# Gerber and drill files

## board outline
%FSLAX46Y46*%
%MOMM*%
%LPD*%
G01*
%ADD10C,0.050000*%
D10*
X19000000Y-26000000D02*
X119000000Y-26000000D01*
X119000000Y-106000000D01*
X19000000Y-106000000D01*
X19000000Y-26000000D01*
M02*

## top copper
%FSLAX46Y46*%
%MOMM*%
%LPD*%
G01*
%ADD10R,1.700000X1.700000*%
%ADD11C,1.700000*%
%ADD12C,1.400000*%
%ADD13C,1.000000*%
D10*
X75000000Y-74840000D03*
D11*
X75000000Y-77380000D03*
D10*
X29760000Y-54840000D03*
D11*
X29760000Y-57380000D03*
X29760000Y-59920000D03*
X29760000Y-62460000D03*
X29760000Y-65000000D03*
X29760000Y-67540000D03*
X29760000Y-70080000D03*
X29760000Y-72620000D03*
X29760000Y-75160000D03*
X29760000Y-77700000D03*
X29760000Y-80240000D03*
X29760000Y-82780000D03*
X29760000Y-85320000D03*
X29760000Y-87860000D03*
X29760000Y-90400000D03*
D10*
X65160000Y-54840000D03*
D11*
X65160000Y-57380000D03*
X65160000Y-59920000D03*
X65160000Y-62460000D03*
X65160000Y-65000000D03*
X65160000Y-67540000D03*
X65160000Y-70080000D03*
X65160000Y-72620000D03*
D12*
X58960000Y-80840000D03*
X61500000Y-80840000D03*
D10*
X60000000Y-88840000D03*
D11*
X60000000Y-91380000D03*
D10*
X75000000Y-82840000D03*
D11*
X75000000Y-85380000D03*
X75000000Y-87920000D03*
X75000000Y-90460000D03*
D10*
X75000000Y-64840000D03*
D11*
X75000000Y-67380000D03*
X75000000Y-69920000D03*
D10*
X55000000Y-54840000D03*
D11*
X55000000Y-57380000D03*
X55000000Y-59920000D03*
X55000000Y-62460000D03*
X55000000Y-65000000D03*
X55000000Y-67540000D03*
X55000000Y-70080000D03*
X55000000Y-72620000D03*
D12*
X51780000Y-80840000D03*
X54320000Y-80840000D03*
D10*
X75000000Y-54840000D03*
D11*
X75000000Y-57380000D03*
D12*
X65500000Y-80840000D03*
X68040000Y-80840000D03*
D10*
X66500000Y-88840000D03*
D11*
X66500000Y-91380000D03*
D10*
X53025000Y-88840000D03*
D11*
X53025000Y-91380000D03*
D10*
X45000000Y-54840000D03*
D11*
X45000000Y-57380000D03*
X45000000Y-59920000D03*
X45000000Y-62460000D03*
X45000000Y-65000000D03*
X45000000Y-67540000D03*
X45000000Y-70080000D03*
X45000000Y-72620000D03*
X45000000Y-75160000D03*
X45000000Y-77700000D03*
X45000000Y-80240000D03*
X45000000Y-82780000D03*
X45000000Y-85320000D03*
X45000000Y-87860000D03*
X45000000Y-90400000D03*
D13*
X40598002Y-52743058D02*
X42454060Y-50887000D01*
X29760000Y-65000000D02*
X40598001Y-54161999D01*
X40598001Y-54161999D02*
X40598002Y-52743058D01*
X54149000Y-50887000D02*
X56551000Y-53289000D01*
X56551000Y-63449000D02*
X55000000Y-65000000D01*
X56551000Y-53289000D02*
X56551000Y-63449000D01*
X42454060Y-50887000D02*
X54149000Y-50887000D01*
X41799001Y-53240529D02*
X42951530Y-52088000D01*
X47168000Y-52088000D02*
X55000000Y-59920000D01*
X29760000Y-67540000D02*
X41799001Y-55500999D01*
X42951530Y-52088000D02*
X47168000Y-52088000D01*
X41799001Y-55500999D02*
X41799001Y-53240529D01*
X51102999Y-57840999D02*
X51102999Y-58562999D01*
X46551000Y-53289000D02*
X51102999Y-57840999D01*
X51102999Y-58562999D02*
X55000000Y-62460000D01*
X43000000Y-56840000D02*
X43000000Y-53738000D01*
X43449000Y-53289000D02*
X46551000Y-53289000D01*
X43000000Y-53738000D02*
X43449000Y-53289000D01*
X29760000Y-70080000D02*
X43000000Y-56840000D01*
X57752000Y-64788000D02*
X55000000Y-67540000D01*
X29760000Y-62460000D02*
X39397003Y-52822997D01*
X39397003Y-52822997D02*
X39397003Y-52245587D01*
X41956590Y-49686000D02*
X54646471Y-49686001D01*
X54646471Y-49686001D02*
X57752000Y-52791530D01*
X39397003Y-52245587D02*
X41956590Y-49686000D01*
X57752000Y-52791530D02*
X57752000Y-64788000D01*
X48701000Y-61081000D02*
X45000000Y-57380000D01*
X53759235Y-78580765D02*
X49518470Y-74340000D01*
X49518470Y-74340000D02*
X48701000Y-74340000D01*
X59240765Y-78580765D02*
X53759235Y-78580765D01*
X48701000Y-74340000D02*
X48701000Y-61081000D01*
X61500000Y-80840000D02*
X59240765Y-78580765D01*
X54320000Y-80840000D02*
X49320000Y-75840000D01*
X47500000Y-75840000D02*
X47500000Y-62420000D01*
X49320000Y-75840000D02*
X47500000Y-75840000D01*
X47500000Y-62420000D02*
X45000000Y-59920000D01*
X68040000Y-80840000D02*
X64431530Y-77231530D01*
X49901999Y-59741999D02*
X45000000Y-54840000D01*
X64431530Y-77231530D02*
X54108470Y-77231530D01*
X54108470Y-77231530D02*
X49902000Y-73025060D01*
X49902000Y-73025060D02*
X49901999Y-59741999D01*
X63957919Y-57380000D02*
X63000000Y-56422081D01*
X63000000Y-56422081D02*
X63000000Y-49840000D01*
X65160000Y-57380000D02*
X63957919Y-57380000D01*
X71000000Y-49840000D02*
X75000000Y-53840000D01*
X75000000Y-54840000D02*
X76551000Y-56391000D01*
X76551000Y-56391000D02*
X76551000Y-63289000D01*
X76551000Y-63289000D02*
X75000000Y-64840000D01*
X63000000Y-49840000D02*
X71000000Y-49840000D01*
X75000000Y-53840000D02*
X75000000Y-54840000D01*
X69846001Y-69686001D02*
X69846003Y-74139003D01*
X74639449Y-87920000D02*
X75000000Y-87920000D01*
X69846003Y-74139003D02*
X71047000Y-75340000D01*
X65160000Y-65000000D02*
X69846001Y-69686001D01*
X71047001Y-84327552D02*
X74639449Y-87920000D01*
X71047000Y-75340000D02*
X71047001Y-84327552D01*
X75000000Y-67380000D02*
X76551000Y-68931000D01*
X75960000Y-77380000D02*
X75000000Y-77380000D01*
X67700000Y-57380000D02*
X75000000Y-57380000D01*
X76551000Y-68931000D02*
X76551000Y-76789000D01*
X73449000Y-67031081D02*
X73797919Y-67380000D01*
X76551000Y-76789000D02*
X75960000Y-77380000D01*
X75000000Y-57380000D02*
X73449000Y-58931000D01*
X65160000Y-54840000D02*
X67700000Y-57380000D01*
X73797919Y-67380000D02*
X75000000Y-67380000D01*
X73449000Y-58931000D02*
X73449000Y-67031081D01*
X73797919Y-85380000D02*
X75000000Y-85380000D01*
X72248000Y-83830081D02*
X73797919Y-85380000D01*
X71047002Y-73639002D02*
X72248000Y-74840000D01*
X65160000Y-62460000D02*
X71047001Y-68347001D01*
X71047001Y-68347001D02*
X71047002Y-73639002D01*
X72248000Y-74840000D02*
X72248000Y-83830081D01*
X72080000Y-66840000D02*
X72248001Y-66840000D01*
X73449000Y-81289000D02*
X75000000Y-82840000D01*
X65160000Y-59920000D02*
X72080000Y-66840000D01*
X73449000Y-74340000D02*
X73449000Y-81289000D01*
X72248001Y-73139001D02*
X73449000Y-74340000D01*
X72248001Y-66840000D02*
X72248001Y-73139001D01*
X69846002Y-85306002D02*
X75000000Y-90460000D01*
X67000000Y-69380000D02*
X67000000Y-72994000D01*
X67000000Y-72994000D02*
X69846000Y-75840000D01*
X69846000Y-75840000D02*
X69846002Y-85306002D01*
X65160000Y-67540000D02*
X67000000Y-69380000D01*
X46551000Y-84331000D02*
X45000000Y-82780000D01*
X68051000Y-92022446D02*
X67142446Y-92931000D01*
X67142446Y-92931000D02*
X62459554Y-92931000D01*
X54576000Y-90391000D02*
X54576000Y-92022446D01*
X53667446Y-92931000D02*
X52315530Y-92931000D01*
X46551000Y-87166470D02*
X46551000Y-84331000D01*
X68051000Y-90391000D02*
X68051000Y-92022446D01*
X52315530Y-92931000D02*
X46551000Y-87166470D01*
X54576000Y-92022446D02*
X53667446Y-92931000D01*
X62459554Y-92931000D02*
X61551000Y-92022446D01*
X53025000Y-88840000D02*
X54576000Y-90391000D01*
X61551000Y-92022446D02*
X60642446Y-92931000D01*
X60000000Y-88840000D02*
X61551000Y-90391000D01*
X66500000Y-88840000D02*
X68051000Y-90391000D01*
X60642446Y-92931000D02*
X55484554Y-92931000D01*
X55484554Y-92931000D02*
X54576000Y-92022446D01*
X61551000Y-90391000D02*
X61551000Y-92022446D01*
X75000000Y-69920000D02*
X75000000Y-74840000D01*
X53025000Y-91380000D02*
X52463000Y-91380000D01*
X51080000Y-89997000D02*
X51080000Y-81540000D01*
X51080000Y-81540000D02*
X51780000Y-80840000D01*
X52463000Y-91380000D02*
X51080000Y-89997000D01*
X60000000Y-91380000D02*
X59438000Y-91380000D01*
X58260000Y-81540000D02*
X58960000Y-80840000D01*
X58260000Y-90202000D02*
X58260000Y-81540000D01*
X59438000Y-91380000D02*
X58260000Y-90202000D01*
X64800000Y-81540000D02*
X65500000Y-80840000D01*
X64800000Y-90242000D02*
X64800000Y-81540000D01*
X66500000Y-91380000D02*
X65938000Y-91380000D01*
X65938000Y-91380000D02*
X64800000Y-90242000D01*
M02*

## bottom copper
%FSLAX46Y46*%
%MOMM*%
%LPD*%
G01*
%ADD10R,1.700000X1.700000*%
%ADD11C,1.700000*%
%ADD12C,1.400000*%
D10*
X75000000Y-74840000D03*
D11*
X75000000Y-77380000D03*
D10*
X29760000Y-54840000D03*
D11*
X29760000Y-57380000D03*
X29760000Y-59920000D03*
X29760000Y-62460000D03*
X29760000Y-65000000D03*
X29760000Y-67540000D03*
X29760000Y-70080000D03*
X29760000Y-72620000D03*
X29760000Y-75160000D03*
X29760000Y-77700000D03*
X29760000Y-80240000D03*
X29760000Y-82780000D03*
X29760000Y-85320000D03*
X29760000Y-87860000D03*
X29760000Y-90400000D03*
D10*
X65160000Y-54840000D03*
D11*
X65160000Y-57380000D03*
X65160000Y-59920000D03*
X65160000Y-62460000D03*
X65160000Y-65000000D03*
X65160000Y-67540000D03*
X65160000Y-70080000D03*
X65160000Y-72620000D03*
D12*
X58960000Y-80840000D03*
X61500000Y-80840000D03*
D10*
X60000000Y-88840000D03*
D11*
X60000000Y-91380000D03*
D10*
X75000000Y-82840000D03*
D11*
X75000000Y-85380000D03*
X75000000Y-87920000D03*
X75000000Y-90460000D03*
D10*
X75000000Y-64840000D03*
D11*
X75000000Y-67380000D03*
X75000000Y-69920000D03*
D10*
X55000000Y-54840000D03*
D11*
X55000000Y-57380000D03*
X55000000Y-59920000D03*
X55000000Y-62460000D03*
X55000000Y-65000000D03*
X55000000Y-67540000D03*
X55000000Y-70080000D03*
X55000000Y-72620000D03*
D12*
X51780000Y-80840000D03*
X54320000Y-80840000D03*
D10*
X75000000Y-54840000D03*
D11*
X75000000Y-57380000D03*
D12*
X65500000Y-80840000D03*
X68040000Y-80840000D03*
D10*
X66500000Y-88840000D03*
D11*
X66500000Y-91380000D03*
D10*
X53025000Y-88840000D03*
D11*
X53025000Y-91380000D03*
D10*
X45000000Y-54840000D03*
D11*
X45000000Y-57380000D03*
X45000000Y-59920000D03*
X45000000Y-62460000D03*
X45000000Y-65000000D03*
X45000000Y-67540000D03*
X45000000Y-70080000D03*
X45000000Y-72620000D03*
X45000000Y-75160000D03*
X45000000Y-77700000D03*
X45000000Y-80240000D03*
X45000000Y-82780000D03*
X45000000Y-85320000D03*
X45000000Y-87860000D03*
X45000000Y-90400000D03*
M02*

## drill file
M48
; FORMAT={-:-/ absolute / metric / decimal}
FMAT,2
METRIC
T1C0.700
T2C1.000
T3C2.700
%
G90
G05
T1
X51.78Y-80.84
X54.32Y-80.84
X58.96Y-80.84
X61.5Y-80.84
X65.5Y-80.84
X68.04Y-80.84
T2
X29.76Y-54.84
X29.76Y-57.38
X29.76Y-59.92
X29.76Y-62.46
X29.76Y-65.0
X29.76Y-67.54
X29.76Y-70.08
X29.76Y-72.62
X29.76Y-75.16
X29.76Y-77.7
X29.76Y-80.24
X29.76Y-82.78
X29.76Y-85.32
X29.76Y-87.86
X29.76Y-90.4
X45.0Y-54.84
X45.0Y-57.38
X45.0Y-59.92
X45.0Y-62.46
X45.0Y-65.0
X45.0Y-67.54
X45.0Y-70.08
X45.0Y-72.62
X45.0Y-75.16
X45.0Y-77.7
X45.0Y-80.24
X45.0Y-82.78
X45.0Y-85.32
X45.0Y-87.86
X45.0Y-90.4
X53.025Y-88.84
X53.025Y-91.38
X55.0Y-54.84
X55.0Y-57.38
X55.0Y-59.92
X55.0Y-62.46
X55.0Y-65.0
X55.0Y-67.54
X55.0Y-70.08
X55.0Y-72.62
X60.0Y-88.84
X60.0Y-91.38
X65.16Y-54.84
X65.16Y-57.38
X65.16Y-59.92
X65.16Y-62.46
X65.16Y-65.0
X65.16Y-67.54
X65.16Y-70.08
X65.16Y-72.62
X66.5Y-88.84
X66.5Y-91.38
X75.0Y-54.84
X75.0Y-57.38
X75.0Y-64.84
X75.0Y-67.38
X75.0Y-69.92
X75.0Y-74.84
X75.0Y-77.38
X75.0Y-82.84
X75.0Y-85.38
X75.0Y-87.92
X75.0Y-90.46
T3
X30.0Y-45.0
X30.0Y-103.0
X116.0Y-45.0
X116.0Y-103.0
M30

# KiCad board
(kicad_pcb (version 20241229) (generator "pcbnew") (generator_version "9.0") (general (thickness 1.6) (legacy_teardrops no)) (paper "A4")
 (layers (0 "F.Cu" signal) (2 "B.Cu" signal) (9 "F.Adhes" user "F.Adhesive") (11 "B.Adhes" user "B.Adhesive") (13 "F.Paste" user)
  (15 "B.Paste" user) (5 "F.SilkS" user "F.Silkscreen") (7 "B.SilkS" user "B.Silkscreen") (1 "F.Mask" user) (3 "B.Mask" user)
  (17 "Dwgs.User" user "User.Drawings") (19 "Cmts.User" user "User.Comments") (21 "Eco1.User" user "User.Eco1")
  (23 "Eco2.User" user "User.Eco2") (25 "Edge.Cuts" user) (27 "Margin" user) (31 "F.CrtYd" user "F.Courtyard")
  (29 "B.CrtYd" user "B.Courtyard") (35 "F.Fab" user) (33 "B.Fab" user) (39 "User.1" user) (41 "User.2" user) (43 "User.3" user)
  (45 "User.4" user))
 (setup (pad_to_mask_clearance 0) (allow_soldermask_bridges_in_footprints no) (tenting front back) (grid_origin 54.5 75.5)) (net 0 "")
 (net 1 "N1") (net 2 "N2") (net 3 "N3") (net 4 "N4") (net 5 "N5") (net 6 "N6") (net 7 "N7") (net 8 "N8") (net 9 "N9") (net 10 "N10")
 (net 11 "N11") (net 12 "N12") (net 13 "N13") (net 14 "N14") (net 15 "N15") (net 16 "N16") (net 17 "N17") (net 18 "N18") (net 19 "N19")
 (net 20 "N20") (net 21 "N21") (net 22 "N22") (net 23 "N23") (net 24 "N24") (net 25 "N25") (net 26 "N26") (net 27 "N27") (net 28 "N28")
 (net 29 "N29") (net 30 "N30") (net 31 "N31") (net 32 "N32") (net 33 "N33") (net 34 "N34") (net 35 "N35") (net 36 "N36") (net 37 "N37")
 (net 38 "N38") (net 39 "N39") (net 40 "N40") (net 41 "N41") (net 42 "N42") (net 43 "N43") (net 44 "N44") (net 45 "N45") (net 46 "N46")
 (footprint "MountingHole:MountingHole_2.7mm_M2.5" (layer "F.Cu") (at 30 103)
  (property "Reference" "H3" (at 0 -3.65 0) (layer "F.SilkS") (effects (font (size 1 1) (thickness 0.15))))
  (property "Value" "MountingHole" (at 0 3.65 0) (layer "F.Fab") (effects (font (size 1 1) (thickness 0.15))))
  (pad "" np_thru_hole circle (at 0 0) (size 2.7 2.7) (drill 2.7) (layers "*.Cu" "*.Mask")))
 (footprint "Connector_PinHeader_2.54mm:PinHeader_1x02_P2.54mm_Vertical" (layer "F.Cu") (at 75 74.84)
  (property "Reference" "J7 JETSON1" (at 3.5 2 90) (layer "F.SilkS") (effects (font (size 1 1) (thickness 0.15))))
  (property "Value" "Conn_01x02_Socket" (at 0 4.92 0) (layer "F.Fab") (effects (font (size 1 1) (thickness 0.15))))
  (pad "1" thru_hole rect (at 0 0) (size 1.7 1.7) (drill 1) (layers "*.Cu" "*.Mask") (remove_unused_layers no) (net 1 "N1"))
  (pad "2" thru_hole circle (at 0 2.54) (size 1.7 1.7) (drill 1) (layers "*.Cu" "*.Mask") (remove_unused_layers no) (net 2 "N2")))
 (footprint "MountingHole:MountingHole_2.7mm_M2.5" (layer "F.Cu") (at 30 45)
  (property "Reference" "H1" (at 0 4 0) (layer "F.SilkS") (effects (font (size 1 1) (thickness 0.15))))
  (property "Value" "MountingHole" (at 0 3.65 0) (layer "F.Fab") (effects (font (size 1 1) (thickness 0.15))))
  (pad "" np_thru_hole circle (at 0 0) (size 2.7 2.7) (drill 2.7) (layers "*.Cu" "*.Mask")))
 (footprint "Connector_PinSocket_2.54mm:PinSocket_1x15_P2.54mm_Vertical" (layer "F.Cu") (at 29.76 54.84)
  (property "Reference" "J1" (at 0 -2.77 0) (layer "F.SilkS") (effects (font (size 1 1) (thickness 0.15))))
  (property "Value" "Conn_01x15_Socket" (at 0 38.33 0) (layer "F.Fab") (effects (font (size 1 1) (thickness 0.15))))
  (pad "1" thru_hole rect (at 0 0) (size 1.7 1.7) (drill 1) (layers "*.Cu" "*.Mask") (remove_unused_layers no) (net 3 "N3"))
  (pad "2" thru_hole circle (at 0 2.54) (size 1.7 1.7) (drill 1) (layers "*.Cu" "*.Mask") (remove_unused_layers no) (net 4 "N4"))
  (pad "3" thru_hole circle (at 0 5.08) (size 1.7 1.7) (drill 1) (layers "*.Cu" "*.Mask") (remove_unused_layers no) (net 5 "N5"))
  (pad "4" thru_hole circle (at 0 7.62) (size 1.7 1.7) (drill 1) (layers "*.Cu" "*.Mask") (remove_unused_layers no) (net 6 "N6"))
  (pad "5" thru_hole circle (at 0 10.16) (size 1.7 1.7) (drill 1) (layers "*.Cu" "*.Mask") (remove_unused_layers no) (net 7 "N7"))
  (pad "6" thru_hole circle (at 0 12.7) (size 1.7 1.7) (drill 1) (layers "*.Cu" "*.Mask") (remove_unused_layers no) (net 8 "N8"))
  (pad "7" thru_hole circle (at 0 15.24) (size 1.7 1.7) (drill 1) (layers "*.Cu" "*.Mask") (remove_unused_layers no) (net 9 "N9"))
  (pad "8" thru_hole circle (at 0 17.78) (size 1.7 1.7) (drill 1) (layers "*.Cu" "*.Mask") (remove_unused_layers no) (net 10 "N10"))
  (pad "9" thru_hole circle (at 0 20.32) (size 1.7 1.7) (drill 1) (layers "*.Cu" "*.Mask") (remove_unused_layers no) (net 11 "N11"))
  (pad "10" thru_hole circle (at 0 22.86) (size 1.7 1.7) (drill 1) (layers "*.Cu" "*.Mask") (remove_unused_layers no) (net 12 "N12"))
  (pad "11" thru_hole circle (at 0 25.4) (size 1.7 1.7) (drill 1) (layers "*.Cu" "*.Mask") (remove_unused_layers no) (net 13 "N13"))
  (pad "12" thru_hole circle (at 0 27.94) (size 1.7 1.7) (drill 1) (layers "*.Cu" "*.Mask") (remove_unused_layers no) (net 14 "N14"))
  (pad "13" thru_hole circle (at 0 30.48) (size 1.7 1.7) (drill 1) (layers "*.Cu" "*.Mask") (remove_unused_layers no) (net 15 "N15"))
  (pad "14" thru_hole circle (at 0 33.02) (size 1.7 1.7) (drill 1) (layers "*.Cu" "*.Mask") (remove_unused_layers no) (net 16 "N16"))
  (pad "15" thru_hole circle (at 0 35.56) (size 1.7 1.7) (drill 1) (layers "*.Cu" "*.Mask") (remove_unused_layers no) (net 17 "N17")))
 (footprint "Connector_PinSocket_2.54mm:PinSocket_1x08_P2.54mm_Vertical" (layer "F.Cu") (at 65.16 54.84)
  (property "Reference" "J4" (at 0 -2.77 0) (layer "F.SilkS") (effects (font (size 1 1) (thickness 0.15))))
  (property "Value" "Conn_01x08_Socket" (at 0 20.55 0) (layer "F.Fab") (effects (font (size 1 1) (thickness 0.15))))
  (pad "1" thru_hole rect (at 0 0) (size 1.7 1.7) (drill 1) (layers "*.Cu" "*.Mask") (remove_unused_layers no) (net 2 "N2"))
  (pad "2" thru_hole circle (at 0 2.54) (size 1.7 1.7) (drill 1) (layers "*.Cu" "*.Mask") (remove_unused_layers no) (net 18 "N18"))
  (pad "3" thru_hole circle (at 0 5.08) (size 1.7 1.7) (drill 1) (layers "*.Cu" "*.Mask") (remove_unused_layers no) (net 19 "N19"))
  (pad "4" thru_hole circle (at 0 7.62) (size 1.7 1.7) (drill 1) (layers "*.Cu" "*.Mask") (remove_unused_layers no) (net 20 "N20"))
  (pad "5" thru_hole circle (at 0 10.16) (size 1.7 1.7) (drill 1) (layers "*.Cu" "*.Mask") (remove_unused_layers no) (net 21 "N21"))
  (pad "6" thru_hole circle (at 0 12.7) (size 1.7 1.7) (drill 1) (layers "*.Cu" "*.Mask") (remove_unused_layers no) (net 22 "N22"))
  (pad "7" thru_hole circle (at 0 15.24) (size 1.7 1.7) (drill 1) (layers "*.Cu" "*.Mask") (remove_unused_layers no) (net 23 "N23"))
  (pad "8" thru_hole circle (at 0 17.78) (size 1.7 1.7) (drill 1) (layers "*.Cu" "*.Mask") (remove_unused_layers no) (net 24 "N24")))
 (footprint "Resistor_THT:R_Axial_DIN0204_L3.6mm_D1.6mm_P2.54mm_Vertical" (layer "F.Cu") (at 58.96 80.84)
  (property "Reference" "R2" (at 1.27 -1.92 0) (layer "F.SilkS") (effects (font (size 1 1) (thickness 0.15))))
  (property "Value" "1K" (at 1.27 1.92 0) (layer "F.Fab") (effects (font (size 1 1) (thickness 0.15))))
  (pad "1" thru_hole circle (at 0 0) (size 1.4 1.4) (drill 0.7) (layers "*.Cu" "*.Mask") (remove_unused_layers no) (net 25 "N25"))
  (pad "2" thru_hole circle (at 2.54 0) (size 1.4 1.4) (drill 0.7) (layers "*.Cu" "*.Mask") (remove_unused_layers no) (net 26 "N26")))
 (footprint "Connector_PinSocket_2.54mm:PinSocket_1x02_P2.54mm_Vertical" (layer "F.Cu") (at 60 88.84)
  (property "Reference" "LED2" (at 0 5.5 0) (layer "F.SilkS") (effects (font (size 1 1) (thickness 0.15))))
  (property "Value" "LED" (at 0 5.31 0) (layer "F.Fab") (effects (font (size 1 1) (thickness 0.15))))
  (pad "1" thru_hole rect (at 0 0) (size 1.7 1.7) (drill 1) (layers "*.Cu" "*.Mask") (remove_unused_layers no) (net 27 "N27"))
  (pad "2" thru_hole circle (at 0 2.54) (size 1.7 1.7) (drill 1) (layers "*.Cu" "*.Mask") (remove_unused_layers no) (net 25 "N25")))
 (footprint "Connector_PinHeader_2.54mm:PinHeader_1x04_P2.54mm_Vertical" (layer "F.Cu") (at 75 82.84)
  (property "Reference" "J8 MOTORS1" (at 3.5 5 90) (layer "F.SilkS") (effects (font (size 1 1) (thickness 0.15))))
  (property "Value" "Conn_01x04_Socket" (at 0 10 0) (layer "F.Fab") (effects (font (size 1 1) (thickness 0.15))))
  (pad "1" thru_hole rect (at 0 0) (size 1.7 1.7) (drill 1) (layers "*.Cu" "*.Mask") (remove_unused_layers no) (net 19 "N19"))
  (pad "2" thru_hole circle (at 0 2.54) (size 1.7 1.7) (drill 1) (layers "*.Cu" "*.Mask") (remove_unused_layers no) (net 20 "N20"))
  (pad "3" thru_hole circle (at 0 5.08) (size 1.7 1.7) (drill 1) (layers "*.Cu" "*.Mask") (remove_unused_layers no) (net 21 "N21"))
  (pad "4" thru_hole circle (at 0 7.62) (size 1.7 1.7) (drill 1) (layers "*.Cu" "*.Mask") (remove_unused_layers no) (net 22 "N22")))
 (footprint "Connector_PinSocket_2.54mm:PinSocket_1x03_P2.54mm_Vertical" (layer "F.Cu") (at 75 64.84)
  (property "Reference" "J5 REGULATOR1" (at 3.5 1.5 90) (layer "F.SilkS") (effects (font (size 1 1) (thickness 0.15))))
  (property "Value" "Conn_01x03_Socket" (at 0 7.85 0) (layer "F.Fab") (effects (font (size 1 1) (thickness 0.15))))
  (pad "1" thru_hole rect (at 0 0) (size 1.7 1.7) (drill 1) (layers "*.Cu" "*.Mask") (remove_unused_layers no) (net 18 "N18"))
  (pad "2" thru_hole circle (at 0 2.54) (size 1.7 1.7) (drill 1) (layers "*.Cu" "*.Mask") (remove_unused_layers no) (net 2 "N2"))
  (pad "3" thru_hole circle (at 0 5.08) (size 1.7 1.7) (drill 1) (layers "*.Cu" "*.Mask") (remove_unused_layers no) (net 1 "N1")))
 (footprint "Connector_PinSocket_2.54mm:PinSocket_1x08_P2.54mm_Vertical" (layer "F.Cu") (at 55 54.84)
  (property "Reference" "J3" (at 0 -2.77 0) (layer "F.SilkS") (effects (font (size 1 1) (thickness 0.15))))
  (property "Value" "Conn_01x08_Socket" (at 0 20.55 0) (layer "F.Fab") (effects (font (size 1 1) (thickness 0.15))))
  (pad "1" thru_hole rect (at 0 0) (size 1.7 1.7) (drill 1) (layers "*.Cu" "*.Mask") (remove_unused_layers no) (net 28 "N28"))
  (pad "2" thru_hole circle (at 0 2.54) (size 1.7 1.7) (drill 1) (layers "*.Cu" "*.Mask") (remove_unused_layers no) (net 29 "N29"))
  (pad "3" thru_hole circle (at 0 5.08) (size 1.7 1.7) (drill 1) (layers "*.Cu" "*.Mask") (remove_unused_layers no) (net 8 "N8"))
  (pad "4" thru_hole circle (at 0 7.62) (size 1.7 1.7) (drill 1) (layers "*.Cu" "*.Mask") (remove_unused_layers no) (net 9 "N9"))
  (pad "5" thru_hole circle (at 0 10.16) (size 1.7 1.7) (drill 1) (layers "*.Cu" "*.Mask") (remove_unused_layers no) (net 7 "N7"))
  (pad "6" thru_hole circle (at 0 12.7) (size 1.7 1.7) (drill 1) (layers "*.Cu" "*.Mask") (remove_unused_layers no) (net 6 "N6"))
  (pad "7" thru_hole circle (at 0 15.24) (size 1.7 1.7) (drill 1) (layers "*.Cu" "*.Mask") (remove_unused_layers no) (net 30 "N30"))
  (pad "8" thru_hole circle (at 0 17.78) (size 1.7 1.7) (drill 1) (layers "*.Cu" "*.Mask") (remove_unused_layers no) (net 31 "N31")))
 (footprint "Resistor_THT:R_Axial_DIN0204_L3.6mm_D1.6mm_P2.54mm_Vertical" (layer "F.Cu") (at 51.78 80.84)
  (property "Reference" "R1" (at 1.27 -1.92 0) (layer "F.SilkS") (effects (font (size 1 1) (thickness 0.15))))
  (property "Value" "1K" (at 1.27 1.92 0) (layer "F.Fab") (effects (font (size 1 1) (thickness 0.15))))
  (pad "1" thru_hole circle (at 0 0) (size 1.4 1.4) (drill 0.7) (layers "*.Cu" "*.Mask") (remove_unused_layers no) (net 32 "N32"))
  (pad "2" thru_hole circle (at 2.54 0) (size 1.4 1.4) (drill 0.7) (layers "*.Cu" "*.Mask") (remove_unused_layers no) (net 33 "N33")))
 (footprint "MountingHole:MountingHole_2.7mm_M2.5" (layer "F.Cu") (at 116 45)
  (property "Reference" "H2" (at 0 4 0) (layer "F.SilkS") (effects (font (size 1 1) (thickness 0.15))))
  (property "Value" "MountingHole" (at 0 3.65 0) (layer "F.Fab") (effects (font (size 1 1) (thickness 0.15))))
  (pad "" np_thru_hole circle (at 0 0) (size 2.7 2.7) (drill 2.7) (layers "*.Cu" "*.Mask")))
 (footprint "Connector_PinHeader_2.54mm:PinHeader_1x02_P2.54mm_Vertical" (layer "F.Cu") (at 75 54.84)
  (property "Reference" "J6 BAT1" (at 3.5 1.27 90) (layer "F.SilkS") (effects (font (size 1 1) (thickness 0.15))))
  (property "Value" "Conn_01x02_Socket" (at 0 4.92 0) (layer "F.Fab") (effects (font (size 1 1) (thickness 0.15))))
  (pad "1" thru_hole rect (at 0 0) (size 1.7 1.7) (drill 1) (layers "*.Cu" "*.Mask") (remove_unused_layers no) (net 18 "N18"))
  (pad "2" thru_hole circle (at 0 2.54) (size 1.7 1.7) (drill 1) (layers "*.Cu" "*.Mask") (remove_unused_layers no) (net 2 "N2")))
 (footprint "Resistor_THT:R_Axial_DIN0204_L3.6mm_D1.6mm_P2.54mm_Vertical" (layer "F.Cu") (at 65.5 80.84)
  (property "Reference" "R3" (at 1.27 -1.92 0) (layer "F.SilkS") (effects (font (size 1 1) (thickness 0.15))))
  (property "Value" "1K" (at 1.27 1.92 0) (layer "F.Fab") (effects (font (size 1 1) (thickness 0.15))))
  (pad "1" thru_hole circle (at 0 0) (size 1.4 1.4) (drill 0.7) (layers "*.Cu" "*.Mask") (remove_unused_layers no) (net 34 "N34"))
  (pad "2" thru_hole circle (at 2.54 0) (size 1.4 1.4) (drill 0.7) (layers "*.Cu" "*.Mask") (remove_unused_layers no) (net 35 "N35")))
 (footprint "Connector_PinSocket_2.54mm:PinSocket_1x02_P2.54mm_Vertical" (layer "F.Cu") (at 66.5 88.84)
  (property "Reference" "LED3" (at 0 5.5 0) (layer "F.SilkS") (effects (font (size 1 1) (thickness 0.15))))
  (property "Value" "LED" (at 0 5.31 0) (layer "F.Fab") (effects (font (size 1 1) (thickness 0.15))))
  (pad "1" thru_hole rect (at 0 0) (size 1.7 1.7) (drill 1) (layers "*.Cu" "*.Mask") (remove_unused_layers no) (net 27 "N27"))
  (pad "2" thru_hole circle (at 0 2.54) (size 1.7 1.7) (drill 1) (layers "*.Cu" "*.Mask") (remove_unused_layers no) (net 34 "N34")))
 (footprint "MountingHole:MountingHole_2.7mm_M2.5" (layer "F.Cu") (at 116 103)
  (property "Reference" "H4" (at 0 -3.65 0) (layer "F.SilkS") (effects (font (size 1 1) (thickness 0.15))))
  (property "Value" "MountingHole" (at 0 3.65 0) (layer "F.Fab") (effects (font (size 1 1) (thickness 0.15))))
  (pad "" np_thru_hole circle (at 0 0) (size 2.7 2.7) (drill 2.7) (layers "*.Cu" "*.Mask")))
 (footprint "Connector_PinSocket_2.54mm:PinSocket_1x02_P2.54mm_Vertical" (layer "F.Cu") (at 53.025 88.84)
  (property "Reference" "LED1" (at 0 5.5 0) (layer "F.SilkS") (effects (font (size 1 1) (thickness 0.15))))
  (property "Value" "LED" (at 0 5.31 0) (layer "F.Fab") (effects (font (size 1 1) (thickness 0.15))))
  (pad "1" thru_hole rect (at 0 0) (size 1.7 1.7) (drill 1) (layers "*.Cu" "*.Mask") (remove_unused_layers no) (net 27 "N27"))
  (pad "2" thru_hole circle (at 0 2.54) (size 1.7 1.7) (drill 1) (layers "*.Cu" "*.Mask") (remove_unused_layers no) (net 32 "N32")))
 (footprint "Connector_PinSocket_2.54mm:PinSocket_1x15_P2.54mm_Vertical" (layer "F.Cu") (at 45 54.84)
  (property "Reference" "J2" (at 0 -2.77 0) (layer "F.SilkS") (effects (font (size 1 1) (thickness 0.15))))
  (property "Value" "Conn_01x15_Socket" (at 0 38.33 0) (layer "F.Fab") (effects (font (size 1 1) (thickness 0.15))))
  (pad "1" thru_hole rect (at 0 0) (size 1.7 1.7) (drill 1) (layers "*.Cu" "*.Mask") (remove_unused_layers no) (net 35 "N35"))
  (pad "2" thru_hole circle (at 0 2.54) (size 1.7 1.7) (drill 1) (layers "*.Cu" "*.Mask") (remove_unused_layers no) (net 26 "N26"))
  (pad "3" thru_hole circle (at 0 5.08) (size 1.7 1.7) (drill 1) (layers "*.Cu" "*.Mask") (remove_unused_layers no) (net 33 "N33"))
  (pad "4" thru_hole circle (at 0 7.62) (size 1.7 1.7) (drill 1) (layers "*.Cu" "*.Mask") (remove_unused_layers no) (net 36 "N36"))
  (pad "5" thru_hole circle (at 0 10.16) (size 1.7 1.7) (drill 1) (layers "*.Cu" "*.Mask") (remove_unused_layers no) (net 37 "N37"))
  (pad "6" thru_hole circle (at 0 12.7) (size 1.7 1.7) (drill 1) (layers "*.Cu" "*.Mask") (remove_unused_layers no) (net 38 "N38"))
  (pad "7" thru_hole circle (at 0 15.24) (size 1.7 1.7) (drill 1) (layers "*.Cu" "*.Mask") (remove_unused_layers no) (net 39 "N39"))
  (pad "8" thru_hole circle (at 0 17.78) (size 1.7 1.7) (drill 1) (layers "*.Cu" "*.Mask") (remove_unused_layers no) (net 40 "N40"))
  (pad "9" thru_hole circle (at 0 20.32) (size 1.7 1.7) (drill 1) (layers "*.Cu" "*.Mask") (remove_unused_layers no) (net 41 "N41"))
  (pad "10" thru_hole circle (at 0 22.86) (size 1.7 1.7) (drill 1) (layers "*.Cu" "*.Mask") (remove_unused_layers no) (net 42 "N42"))
  (pad "11" thru_hole circle (at 0 25.4) (size 1.7 1.7) (drill 1) (layers "*.Cu" "*.Mask") (remove_unused_layers no) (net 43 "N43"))
  (pad "12" thru_hole circle (at 0 27.94) (size 1.7 1.7) (drill 1) (layers "*.Cu" "*.Mask") (remove_unused_layers no) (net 27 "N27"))
  (pad "13" thru_hole circle (at 0 30.48) (size 1.7 1.7) (drill 1) (layers "*.Cu" "*.Mask") (remove_unused_layers no) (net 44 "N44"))
  (pad "14" thru_hole circle (at 0 33.02) (size 1.7 1.7) (drill 1) (layers "*.Cu" "*.Mask") (remove_unused_layers no) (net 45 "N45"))
  (pad "15" thru_hole circle (at 0 35.56) (size 1.7 1.7) (drill 1) (layers "*.Cu" "*.Mask") (remove_unused_layers no) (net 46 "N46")))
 (gr_rect (start 19 26) (end 119 106) (stroke (width 0.05) (type default)) (fill no) (layer "Edge.Cuts"))
 (segment (start 40.598002 52.743058) (end 42.45406 50.887) (width 1) (layer "F.Cu") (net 7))
 (segment (start 29.76 65) (end 40.598001 54.161999) (width 1) (layer "F.Cu") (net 7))
 (segment (start 40.598001 54.161999) (end 40.598002 52.743058) (width 1) (layer "F.Cu") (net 7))
 (segment (start 54.149 50.887) (end 56.551 53.289) (width 1) (layer "F.Cu") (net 7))
 (segment (start 56.551 63.449) (end 55 65) (width 1) (layer "F.Cu") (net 7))
 (segment (start 56.551 53.289) (end 56.551 63.449) (width 1) (layer "F.Cu") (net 7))
 (segment (start 42.45406 50.887) (end 54.149 50.887) (width 1) (layer "F.Cu") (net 7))
 (segment (start 41.799001 53.240529) (end 42.95153 52.088) (width 1) (layer "F.Cu") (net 8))
 (segment (start 47.168 52.088) (end 55 59.92) (width 1) (layer "F.Cu") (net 8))
 (segment (start 29.76 67.54) (end 41.799001 55.500999) (width 1) (layer "F.Cu") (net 8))
 (segment (start 42.95153 52.088) (end 47.168 52.088) (width 1) (layer "F.Cu") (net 8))
 (segment (start 41.799001 55.500999) (end 41.799001 53.240529) (width 1) (layer "F.Cu") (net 8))
 (segment (start 51.102999 57.840999) (end 51.102999 58.562999) (width 1) (layer "F.Cu") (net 9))
 (segment (start 46.551 53.289) (end 51.102999 57.840999) (width 1) (layer "F.Cu") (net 9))
 (segment (start 51.102999 58.562999) (end 55 62.46) (width 1) (layer "F.Cu") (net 9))
 (segment (start 43 56.84) (end 43 53.738) (width 1) (layer "F.Cu") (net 9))
 (segment (start 43.449 53.289) (end 46.551 53.289) (width 1) (layer "F.Cu") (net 9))
 (segment (start 43 53.738) (end 43.449 53.289) (width 1) (layer "F.Cu") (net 9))
 (segment (start 29.76 70.08) (end 43 56.84) (width 1) (layer "F.Cu") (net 9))
 (segment (start 57.752 64.788) (end 55 67.54) (width 1) (layer "F.Cu") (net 6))
 (segment (start 29.76 62.46) (end 39.397003 52.822997) (width 1) (layer "F.Cu") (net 6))
 (segment (start 39.397003 52.822997) (end 39.397003 52.245587) (width 1) (layer "F.Cu") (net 6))
 (segment (start 41.95659 49.686) (end 54.646471 49.686001) (width 1) (layer "F.Cu") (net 6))
 (segment (start 54.646471 49.686001) (end 57.752 52.79153) (width 1) (layer "F.Cu") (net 6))
 (segment (start 39.397003 52.245587) (end 41.95659 49.686) (width 1) (layer "F.Cu") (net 6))
 (segment (start 57.752 52.79153) (end 57.752 64.788) (width 1) (layer "F.Cu") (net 6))
 (segment (start 48.701 61.081) (end 45 57.38) (width 1) (layer "F.Cu") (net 26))
 (segment (start 53.759235 78.580765) (end 49.51847 74.34) (width 1) (layer "F.Cu") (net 26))
 (segment (start 49.51847 74.34) (end 48.701 74.34) (width 1) (layer "F.Cu") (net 26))
 (segment (start 59.240765 78.580765) (end 53.759235 78.580765) (width 1) (layer "F.Cu") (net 26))
 (segment (start 48.701 74.34) (end 48.701 61.081) (width 1) (layer "F.Cu") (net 26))
 (segment (start 61.5 80.84) (end 59.240765 78.580765) (width 1) (layer "F.Cu") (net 26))
 (segment (start 54.32 80.84) (end 49.32 75.84) (width 1) (layer "F.Cu") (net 33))
 (segment (start 47.5 75.84) (end 47.5 62.42) (width 1) (layer "F.Cu") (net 33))
 (segment (start 49.32 75.84) (end 47.5 75.84) (width 1) (layer "F.Cu") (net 33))
 (segment (start 47.5 62.42) (end 45 59.92) (width 1) (layer "F.Cu") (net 33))
 (segment (start 68.04 80.84) (end 64.43153 77.23153) (width 1) (layer "F.Cu") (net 35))
 (segment (start 49.901999 59.741999) (end 45 54.84) (width 1) (layer "F.Cu") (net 35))
 (segment (start 64.43153 77.23153) (end 54.10847 77.23153) (width 1) (layer "F.Cu") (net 35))
 (segment (start 54.10847 77.23153) (end 49.902 73.02506) (width 1) (layer "F.Cu") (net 35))
 (segment (start 49.902 73.02506) (end 49.901999 59.741999) (width 1) (layer "F.Cu") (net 35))
 (segment (start 63.957919 57.38) (end 63 56.422081) (width 1) (layer "F.Cu") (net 18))
 (segment (start 63 56.422081) (end 63 49.84) (width 1) (layer "F.Cu") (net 18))
 (segment (start 65.16 57.38) (end 63.957919 57.38) (width 1) (layer "F.Cu") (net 18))
 (segment (start 71 49.84) (end 75 53.84) (width 1) (layer "F.Cu") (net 18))
 (segment (start 75 54.84) (end 76.551 56.391) (width 1) (layer "F.Cu") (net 18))
 (segment (start 76.551 56.391) (end 76.551 63.289) (width 1) (layer "F.Cu") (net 18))
 (segment (start 76.551 63.289) (end 75 64.84) (width 1) (layer "F.Cu") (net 18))
 (segment (start 63 49.84) (end 71 49.84) (width 1) (layer "F.Cu") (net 18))
 (segment (start 75 53.84) (end 75 54.84) (width 1) (layer "F.Cu") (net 18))
 (segment (start 69.846001 69.686001) (end 69.846003 74.139003) (width 1) (layer "F.Cu") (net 21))
 (segment (start 74.639449 87.92) (end 75 87.92) (width 1) (layer "F.Cu") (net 21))
 (segment (start 69.846003 74.139003) (end 71.047 75.34) (width 1) (layer "F.Cu") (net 21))
 (segment (start 65.16 65) (end 69.846001 69.686001) (width 1) (layer "F.Cu") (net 21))
 (segment (start 71.047001 84.327552) (end 74.639449 87.92) (width 1) (layer "F.Cu") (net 21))
 (segment (start 71.047 75.34) (end 71.047001 84.327552) (width 1) (layer "F.Cu") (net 21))
 (segment (start 75 67.38) (end 76.551 68.931) (width 1) (layer "F.Cu") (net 2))
 (segment (start 75.96 77.38) (end 75 77.38) (width 1) (layer "F.Cu") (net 2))
 (segment (start 67.7 57.38) (end 75 57.38) (width 1) (layer "F.Cu") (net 2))
 (segment (start 76.551 68.931) (end 76.551 76.789) (width 1) (layer "F.Cu") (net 2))
 (segment (start 73.449 67.031081) (end 73.797919 67.38) (width 1) (layer "F.Cu") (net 2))
 (segment (start 76.551 76.789) (end 75.96 77.38) (width 1) (layer "F.Cu") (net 2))
 (segment (start 75 57.38) (end 73.449 58.931) (width 1) (layer "F.Cu") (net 2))
 (segment (start 65.16 54.84) (end 67.7 57.38) (width 1) (layer "F.Cu") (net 2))
 (segment (start 73.797919 67.38) (end 75 67.38) (width 1) (layer "F.Cu") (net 2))
 (segment (start 73.449 58.931) (end 73.449 67.031081) (width 1) (layer "F.Cu") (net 2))
 (segment (start 73.797919 85.38) (end 75 85.38) (width 1) (layer "F.Cu") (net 20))
 (segment (start 72.248 83.830081) (end 73.797919 85.38) (width 1) (layer "F.Cu") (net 20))
 (segment (start 71.047002 73.639002) (end 72.248 74.84) (width 1) (layer "F.Cu") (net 20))
 (segment (start 65.16 62.46) (end 71.047001 68.347001) (width 1) (layer "F.Cu") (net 20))
 (segment (start 71.047001 68.347001) (end 71.047002 73.639002) (width 1) (layer "F.Cu") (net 20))
 (segment (start 72.248 74.84) (end 72.248 83.830081) (width 1) (layer "F.Cu") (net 20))
 (segment (start 72.08 66.84) (end 72.248001 66.84) (width 1) (layer "F.Cu") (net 19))
 (segment (start 73.449 81.289) (end 75 82.84) (width 1) (layer "F.Cu") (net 19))
 (segment (start 65.16 59.92) (end 72.08 66.84) (width 1) (layer "F.Cu") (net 19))
 (segment (start 73.449 74.34) (end 73.449 81.289) (width 1) (layer "F.Cu") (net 19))
 (segment (start 72.248001 73.139001) (end 73.449 74.34) (width 1) (layer "F.Cu") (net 19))
 (segment (start 72.248001 66.84) (end 72.248001 73.139001) (width 1) (layer "F.Cu") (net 19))
 (segment (start 69.846002 85.306002) (end 75 90.46) (width 1) (layer "F.Cu") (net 22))
 (segment (start 67 69.38) (end 67 72.994) (width 1) (layer "F.Cu") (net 22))
 (segment (start 67 72.994) (end 69.846 75.84) (width 1) (layer "F.Cu") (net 22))
 (segment (start 69.846 75.84) (end 69.846002 85.306002) (width 1) (layer "F.Cu") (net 22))
 (segment (start 65.16 67.54) (end 67 69.38) (width 1) (layer "F.Cu") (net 22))
 (segment (start 46.551 84.331) (end 45 82.78) (width 1) (layer "F.Cu") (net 27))
 (segment (start 68.051 92.022446) (end 67.142446 92.931) (width 1) (layer "F.Cu") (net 27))
 (segment (start 67.142446 92.931) (end 62.459554 92.931) (width 1) (layer "F.Cu") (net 27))
 (segment (start 54.576 90.391) (end 54.576 92.022446) (width 1) (layer "F.Cu") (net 27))
 (segment (start 53.667446 92.931) (end 52.31553 92.931) (width 1) (layer "F.Cu") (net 27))
 (segment (start 46.551 87.16647) (end 46.551 84.331) (width 1) (layer "F.Cu") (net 27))
 (segment (start 68.051 90.391) (end 68.051 92.022446) (width 1) (layer "F.Cu") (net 27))
 (segment (start 52.31553 92.931) (end 46.551 87.16647) (width 1) (layer "F.Cu") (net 27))
 (segment (start 54.576 92.022446) (end 53.667446 92.931) (width 1) (layer "F.Cu") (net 27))
 (segment (start 62.459554 92.931) (end 61.551 92.022446) (width 1) (layer "F.Cu") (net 27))
 (segment (start 53.025 88.84) (end 54.576 90.391) (width 1) (layer "F.Cu") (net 27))
 (segment (start 61.551 92.022446) (end 60.642446 92.931) (width 1) (layer "F.Cu") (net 27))
 (segment (start 60 88.84) (end 61.551 90.391) (width 1) (layer "F.Cu") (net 27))
 (segment (start 66.5 88.84) (end 68.051 90.391) (width 1) (layer "F.Cu") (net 27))
 (segment (start 60.642446 92.931) (end 55.484554 92.931) (width 1) (layer "F.Cu") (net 27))
 (segment (start 55.484554 92.931) (end 54.576 92.022446) (width 1) (layer "F.Cu") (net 27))
 (segment (start 61.551 90.391) (end 61.551 92.022446) (width 1) (layer "F.Cu") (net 27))
 (segment (start 75 69.92) (end 75 74.84) (width 1) (layer "F.Cu") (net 1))
 (segment (start 53.025 91.38) (end 52.463 91.38) (width 1) (layer "F.Cu") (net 32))
 (segment (start 51.08 89.997) (end 51.08 81.54) (width 1) (layer "F.Cu") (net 32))
 (segment (start 51.08 81.54) (end 51.78 80.84) (width 1) (layer "F.Cu") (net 32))
 (segment (start 52.463 91.38) (end 51.08 89.997) (width 1) (layer "F.Cu") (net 32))
 (segment (start 60 91.38) (end 59.438 91.38) (width 1) (layer "F.Cu") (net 25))
 (segment (start 58.26 81.54) (end 58.96 80.84) (width 1) (layer "F.Cu") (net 25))
 (segment (start 58.26 90.202) (end 58.26 81.54) (width 1) (layer "F.Cu") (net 25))
 (segment (start 59.438 91.38) (end 58.26 90.202) (width 1) (layer "F.Cu") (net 25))
 (segment (start 64.8 81.54) (end 65.5 80.84) (width 1) (layer "F.Cu") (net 34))
 (segment (start 64.8 90.242) (end 64.8 81.54) (width 1) (layer "F.Cu") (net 34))
 (segment (start 66.5 91.38) (end 65.938 91.38) (width 1) (layer "F.Cu") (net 34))
 (segment (start 65.938 91.38) (end 64.8 90.242) (width 1) (layer "F.Cu") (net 34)))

